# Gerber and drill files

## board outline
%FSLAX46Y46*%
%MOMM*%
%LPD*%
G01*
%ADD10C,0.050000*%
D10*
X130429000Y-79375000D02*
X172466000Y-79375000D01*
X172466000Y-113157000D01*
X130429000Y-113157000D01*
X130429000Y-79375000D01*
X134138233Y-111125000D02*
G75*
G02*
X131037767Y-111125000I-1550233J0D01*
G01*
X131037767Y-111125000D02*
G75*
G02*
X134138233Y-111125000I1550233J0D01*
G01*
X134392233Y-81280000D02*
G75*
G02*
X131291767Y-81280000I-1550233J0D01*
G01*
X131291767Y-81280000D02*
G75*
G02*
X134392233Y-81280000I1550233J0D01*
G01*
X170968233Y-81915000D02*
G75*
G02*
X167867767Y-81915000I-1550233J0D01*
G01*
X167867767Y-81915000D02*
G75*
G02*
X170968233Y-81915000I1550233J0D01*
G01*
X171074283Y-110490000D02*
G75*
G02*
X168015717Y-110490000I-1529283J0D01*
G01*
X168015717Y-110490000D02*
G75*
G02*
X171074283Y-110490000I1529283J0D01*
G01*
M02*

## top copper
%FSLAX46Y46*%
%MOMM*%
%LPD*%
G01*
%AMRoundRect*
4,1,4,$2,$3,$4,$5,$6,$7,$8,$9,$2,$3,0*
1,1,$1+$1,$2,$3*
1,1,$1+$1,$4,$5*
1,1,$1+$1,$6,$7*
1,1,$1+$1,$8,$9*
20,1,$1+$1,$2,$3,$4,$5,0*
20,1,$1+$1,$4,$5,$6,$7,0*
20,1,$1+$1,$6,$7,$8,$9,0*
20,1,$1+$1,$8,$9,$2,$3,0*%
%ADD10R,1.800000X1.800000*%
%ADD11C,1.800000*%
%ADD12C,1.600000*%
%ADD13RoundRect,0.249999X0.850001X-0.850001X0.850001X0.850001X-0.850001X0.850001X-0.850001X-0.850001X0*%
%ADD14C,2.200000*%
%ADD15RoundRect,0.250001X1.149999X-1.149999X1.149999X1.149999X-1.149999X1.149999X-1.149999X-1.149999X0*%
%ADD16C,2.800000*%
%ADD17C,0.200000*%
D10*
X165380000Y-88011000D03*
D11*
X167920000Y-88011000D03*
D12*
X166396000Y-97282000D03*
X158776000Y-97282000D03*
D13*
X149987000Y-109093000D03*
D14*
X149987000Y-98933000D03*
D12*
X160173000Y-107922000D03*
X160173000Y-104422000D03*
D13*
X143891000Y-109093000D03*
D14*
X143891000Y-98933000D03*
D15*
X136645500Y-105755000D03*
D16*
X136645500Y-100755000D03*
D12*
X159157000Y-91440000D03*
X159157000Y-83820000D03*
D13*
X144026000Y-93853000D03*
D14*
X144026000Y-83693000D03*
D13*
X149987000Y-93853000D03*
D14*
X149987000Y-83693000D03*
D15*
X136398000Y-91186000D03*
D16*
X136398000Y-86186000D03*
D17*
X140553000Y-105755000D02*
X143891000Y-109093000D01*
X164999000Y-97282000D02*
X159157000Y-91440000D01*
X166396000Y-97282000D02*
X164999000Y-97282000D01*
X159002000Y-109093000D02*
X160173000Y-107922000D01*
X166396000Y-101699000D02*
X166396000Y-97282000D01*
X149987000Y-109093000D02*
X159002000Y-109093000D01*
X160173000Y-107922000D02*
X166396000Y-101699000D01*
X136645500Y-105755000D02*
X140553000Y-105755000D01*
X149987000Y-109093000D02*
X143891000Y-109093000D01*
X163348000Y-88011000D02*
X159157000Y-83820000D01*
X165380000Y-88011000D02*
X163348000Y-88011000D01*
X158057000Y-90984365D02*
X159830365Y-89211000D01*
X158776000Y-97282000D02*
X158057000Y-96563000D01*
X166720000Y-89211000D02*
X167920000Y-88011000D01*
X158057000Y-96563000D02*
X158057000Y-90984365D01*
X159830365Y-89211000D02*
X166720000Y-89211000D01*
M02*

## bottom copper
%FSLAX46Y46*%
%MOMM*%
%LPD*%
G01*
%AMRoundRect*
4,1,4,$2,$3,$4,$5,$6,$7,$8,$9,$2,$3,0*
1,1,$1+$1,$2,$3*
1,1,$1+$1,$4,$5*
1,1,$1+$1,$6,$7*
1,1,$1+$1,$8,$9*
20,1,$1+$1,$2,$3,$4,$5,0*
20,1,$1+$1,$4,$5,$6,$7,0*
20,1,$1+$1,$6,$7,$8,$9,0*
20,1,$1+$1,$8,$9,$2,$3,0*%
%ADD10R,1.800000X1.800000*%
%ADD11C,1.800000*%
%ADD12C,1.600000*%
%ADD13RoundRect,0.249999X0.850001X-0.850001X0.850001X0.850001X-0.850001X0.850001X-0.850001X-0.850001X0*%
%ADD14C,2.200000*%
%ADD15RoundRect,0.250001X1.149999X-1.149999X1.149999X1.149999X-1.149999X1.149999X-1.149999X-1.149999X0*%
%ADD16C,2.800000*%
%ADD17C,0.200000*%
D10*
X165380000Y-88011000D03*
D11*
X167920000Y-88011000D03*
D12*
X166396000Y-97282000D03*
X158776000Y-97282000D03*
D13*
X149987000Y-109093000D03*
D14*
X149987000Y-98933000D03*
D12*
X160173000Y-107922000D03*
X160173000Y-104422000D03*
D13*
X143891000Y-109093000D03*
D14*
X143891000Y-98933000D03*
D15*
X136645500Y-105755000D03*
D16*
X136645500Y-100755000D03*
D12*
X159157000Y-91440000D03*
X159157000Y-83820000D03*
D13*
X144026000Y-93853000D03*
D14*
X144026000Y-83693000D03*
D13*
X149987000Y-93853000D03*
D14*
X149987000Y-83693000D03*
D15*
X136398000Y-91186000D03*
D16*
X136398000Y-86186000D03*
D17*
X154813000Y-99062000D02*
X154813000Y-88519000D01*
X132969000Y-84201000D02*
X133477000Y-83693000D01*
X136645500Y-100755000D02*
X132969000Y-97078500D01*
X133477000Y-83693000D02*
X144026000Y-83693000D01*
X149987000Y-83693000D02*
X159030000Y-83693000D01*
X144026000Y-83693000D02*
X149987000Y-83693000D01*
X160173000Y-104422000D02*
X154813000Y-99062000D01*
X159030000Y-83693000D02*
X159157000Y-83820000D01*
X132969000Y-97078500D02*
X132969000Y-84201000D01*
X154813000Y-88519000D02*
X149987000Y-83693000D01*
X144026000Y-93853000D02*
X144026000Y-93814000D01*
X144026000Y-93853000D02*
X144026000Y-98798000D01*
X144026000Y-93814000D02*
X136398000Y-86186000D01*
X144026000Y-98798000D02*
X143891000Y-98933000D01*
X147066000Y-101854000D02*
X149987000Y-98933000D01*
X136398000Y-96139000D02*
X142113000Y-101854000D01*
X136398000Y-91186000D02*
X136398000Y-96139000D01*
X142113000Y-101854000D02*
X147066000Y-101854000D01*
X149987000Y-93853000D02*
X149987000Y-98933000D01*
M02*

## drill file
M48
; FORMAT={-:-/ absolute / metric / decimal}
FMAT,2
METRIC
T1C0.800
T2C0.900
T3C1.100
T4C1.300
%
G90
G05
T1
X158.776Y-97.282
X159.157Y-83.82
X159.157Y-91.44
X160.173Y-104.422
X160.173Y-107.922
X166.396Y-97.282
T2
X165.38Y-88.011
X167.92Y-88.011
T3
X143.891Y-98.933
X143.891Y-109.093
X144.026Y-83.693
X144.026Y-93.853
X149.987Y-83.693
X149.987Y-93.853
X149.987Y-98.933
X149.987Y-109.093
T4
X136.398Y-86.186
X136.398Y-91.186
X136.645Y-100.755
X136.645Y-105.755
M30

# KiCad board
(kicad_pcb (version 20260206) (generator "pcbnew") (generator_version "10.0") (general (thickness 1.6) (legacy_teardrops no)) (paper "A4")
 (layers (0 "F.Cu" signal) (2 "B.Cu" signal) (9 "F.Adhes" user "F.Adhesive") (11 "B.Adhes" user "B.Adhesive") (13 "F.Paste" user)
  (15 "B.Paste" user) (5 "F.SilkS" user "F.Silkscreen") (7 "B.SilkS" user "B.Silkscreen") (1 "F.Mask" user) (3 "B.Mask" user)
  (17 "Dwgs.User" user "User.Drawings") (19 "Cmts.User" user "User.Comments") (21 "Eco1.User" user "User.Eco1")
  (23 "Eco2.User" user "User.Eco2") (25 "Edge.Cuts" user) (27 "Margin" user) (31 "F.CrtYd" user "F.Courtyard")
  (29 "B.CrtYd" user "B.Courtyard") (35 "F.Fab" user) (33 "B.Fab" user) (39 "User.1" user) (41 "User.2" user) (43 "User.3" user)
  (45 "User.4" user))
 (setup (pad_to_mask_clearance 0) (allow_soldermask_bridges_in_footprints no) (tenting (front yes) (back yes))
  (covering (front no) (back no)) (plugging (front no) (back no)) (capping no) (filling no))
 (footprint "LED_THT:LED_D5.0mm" (layer "F.Cu") (at 165.38 88.011)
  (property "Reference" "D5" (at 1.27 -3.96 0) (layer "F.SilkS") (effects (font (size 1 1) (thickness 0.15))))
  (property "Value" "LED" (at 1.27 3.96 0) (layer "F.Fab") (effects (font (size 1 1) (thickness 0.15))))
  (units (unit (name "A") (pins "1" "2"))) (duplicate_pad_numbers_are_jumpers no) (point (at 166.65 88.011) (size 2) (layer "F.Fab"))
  (pad "1" thru_hole rect (at 0 0) (size 1.8 1.8) (drill 0.9) (layers "*.Cu" "*.Mask") (remove_unused_layers no) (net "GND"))
  (pad "2" thru_hole circle (at 2.54 0) (size 1.8 1.8) (drill 0.9) (layers "*.Cu" "*.Mask") (remove_unused_layers no) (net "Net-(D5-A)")))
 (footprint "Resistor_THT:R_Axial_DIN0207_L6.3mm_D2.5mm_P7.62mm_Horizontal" (layer "F.Cu") (at 166.396 97.282 180)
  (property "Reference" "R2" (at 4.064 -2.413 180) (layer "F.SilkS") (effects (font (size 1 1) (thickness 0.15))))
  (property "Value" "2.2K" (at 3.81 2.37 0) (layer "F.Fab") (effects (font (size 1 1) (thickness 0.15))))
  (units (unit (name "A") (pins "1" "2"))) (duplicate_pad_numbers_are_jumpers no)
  (pad "1" thru_hole circle (at 0 0 180) (size 1.6 1.6) (drill 0.8) (layers "*.Cu" "*.Mask") (remove_unused_layers no) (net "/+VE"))
  (pad "2" thru_hole circle (at 7.62 0 180) (size 1.6 1.6) (drill 0.8) (layers "*.Cu" "*.Mask") (remove_unused_layers no) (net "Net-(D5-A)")))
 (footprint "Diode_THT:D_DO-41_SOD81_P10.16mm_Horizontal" (layer "F.Cu") (at 149.987 109.093 90)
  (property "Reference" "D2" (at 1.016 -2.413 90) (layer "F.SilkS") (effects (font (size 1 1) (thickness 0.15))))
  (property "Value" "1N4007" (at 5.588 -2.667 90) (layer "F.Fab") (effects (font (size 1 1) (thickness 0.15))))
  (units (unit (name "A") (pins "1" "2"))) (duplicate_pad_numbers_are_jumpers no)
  (pad "1" thru_hole roundrect (at 0 0 90) (size 2.2 2.2) (drill 1.1) (layers "*.Cu" "*.Mask") (remove_unused_layers no)
   (roundrect_rratio 0.113636) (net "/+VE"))
  (pad "2" thru_hole circle (at 10.16 0 90) (size 2.2 2.2) (drill 1.1) (layers "*.Cu" "*.Mask") (remove_unused_layers no) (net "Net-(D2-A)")))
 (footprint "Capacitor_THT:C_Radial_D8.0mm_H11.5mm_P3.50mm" (layer "F.Cu") (at 160.173 107.922 90)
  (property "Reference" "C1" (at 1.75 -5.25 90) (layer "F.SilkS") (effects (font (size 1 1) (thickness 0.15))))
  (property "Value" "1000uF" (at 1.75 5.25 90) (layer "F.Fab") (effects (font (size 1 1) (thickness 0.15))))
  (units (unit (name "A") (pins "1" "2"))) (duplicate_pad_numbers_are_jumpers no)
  (pad "1" thru_hole circle (at 0 0 90) (size 1.6 1.6) (drill 0.8) (layers "*.Cu" "*.Mask") (remove_unused_layers no) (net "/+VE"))
  (pad "2" thru_hole circle (at 3.5 0 90) (size 1.6 1.6) (drill 0.8) (layers "*.Cu" "*.Mask") (remove_unused_layers no) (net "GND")))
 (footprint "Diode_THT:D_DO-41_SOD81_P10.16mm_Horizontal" (layer "F.Cu") (at 143.891 109.093 90)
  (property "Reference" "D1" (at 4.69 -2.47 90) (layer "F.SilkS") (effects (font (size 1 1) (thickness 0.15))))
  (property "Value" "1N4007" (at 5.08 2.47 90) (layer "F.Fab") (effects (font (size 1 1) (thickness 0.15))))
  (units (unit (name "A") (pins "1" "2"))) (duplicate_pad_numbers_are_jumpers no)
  (pad "1" thru_hole roundrect (at 0 0 90) (size 2.2 2.2) (drill 1.1) (layers "*.Cu" "*.Mask") (remove_unused_layers no)
   (roundrect_rratio 0.113636) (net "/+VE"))
  (pad "2" thru_hole circle (at 10.16 0 90) (size 2.2 2.2) (drill 1.1) (layers "*.Cu" "*.Mask") (remove_unused_layers no) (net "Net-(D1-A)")))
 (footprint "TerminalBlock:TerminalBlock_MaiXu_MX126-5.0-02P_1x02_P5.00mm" (layer "F.Cu") (at 136.6455 105.755 90)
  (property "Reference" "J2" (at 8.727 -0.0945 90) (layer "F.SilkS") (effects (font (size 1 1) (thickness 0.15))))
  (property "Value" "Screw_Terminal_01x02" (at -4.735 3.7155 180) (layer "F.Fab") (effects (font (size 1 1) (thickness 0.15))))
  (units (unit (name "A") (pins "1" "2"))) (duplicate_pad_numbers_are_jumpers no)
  (pad "1" thru_hole roundrect (at 0 0 90) (size 2.8 2.8) (drill 1.3) (layers "*.Cu" "*.Mask") (remove_unused_layers no)
   (roundrect_rratio 0.089286) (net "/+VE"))
  (pad "2" thru_hole circle (at 5 0 90) (size 2.8 2.8) (drill 1.3) (layers "*.Cu" "*.Mask") (remove_unused_layers no) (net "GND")))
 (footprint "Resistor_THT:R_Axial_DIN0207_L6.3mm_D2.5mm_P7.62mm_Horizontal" (layer "F.Cu") (at 159.157 91.44 90)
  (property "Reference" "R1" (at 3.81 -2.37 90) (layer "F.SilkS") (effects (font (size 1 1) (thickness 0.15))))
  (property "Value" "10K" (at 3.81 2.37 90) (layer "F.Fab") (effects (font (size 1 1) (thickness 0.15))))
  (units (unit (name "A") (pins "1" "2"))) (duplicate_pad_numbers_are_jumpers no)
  (pad "1" thru_hole circle (at 0 0 90) (size 1.6 1.6) (drill 0.8) (layers "*.Cu" "*.Mask") (remove_unused_layers no) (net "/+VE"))
  (pad "2" thru_hole circle (at 7.62 0 90) (size 1.6 1.6) (drill 0.8) (layers "*.Cu" "*.Mask") (remove_unused_layers no) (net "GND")))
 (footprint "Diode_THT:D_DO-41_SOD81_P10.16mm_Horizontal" (layer "F.Cu") (at 144.026 93.853 90)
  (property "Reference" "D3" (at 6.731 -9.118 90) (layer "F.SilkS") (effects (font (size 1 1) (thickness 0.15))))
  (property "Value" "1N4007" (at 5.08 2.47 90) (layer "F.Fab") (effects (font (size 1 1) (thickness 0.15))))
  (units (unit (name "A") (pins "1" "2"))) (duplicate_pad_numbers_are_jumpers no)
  (pad "1" thru_hole roundrect (at 0 0 90) (size 2.2 2.2) (drill 1.1) (layers "*.Cu" "*.Mask") (remove_unused_layers no)
   (roundrect_rratio 0.113636) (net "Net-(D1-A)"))
  (pad "2" thru_hole circle (at 10.16 0 90) (size 2.2 2.2) (drill 1.1) (layers "*.Cu" "*.Mask") (remove_unused_layers no) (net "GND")))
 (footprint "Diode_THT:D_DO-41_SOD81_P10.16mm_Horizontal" (layer "F.Cu") (at 149.987 93.853 90)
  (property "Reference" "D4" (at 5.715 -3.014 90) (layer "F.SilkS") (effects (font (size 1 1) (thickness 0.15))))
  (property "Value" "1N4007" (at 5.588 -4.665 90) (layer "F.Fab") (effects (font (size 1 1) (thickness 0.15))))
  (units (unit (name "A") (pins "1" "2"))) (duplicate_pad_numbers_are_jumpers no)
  (pad "1" thru_hole roundrect (at 0 0 90) (size 2.2 2.2) (drill 1.1) (layers "*.Cu" "*.Mask") (remove_unused_layers no)
   (roundrect_rratio 0.113636) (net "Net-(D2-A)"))
  (pad "2" thru_hole circle (at 10.16 0 90) (size 2.2 2.2) (drill 1.1) (layers "*.Cu" "*.Mask") (remove_unused_layers no) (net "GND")))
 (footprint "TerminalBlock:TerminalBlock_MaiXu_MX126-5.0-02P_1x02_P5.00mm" (layer "F.Cu") (at 136.398 91.186 90)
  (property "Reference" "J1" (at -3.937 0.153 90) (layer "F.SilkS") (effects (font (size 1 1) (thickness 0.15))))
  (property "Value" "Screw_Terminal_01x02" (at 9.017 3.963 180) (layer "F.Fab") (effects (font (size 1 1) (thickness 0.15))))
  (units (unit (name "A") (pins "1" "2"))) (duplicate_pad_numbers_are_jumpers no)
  (pad "1" thru_hole roundrect (at 0 0 90) (size 2.8 2.8) (drill 1.3) (layers "*.Cu" "*.Mask") (remove_unused_layers no)
   (roundrect_rratio 0.089286) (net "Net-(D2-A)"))
  (pad "2" thru_hole circle (at 5 0 90) (size 2.8 2.8) (drill 1.3) (layers "*.Cu" "*.Mask") (remove_unused_layers no) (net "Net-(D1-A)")))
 (gr_rect (start 130.429 79.375) (end 172.466 113.157) (stroke (width 0.05) (type default)) (fill no) (layer "Edge.Cuts"))
 (gr_circle (center 132.588 111.125) (end 131.318 112.014) (stroke (width 0.05) (type default)) (fill no) (layer "Edge.Cuts"))
 (gr_circle (center 132.842 81.28) (end 131.572 80.391) (stroke (width 0.05) (type default)) (fill no) (layer "Edge.Cuts"))
 (gr_circle (center 169.418 81.915) (end 168.148 81.026) (stroke (width 0.05) (type default)) (fill no) (layer "Edge.Cuts"))
 (gr_circle (center 169.545 110.49) (end 170.688 111.506) (stroke (width 0.05) (type default)) (fill no) (layer "Edge.Cuts"))
 (segment (start 140.553 105.755) (end 143.891 109.093) (width 0.2) (layer "F.Cu") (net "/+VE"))
 (segment (start 164.999 97.282) (end 159.157 91.44) (width 0.2) (layer "F.Cu") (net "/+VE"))
 (segment (start 166.396 97.282) (end 164.999 97.282) (width 0.2) (layer "F.Cu") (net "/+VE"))
 (segment (start 159.002 109.093) (end 160.173 107.922) (width 0.2) (layer "F.Cu") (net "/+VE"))
 (segment (start 166.396 101.699) (end 166.396 97.282) (width 0.2) (layer "F.Cu") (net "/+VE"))
 (segment (start 149.987 109.093) (end 159.002 109.093) (width 0.2) (layer "F.Cu") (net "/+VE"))
 (segment (start 160.173 107.922) (end 166.396 101.699) (width 0.2) (layer "F.Cu") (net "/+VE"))
 (segment (start 136.6455 105.755) (end 140.553 105.755) (width 0.2) (layer "F.Cu") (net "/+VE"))
 (segment (start 149.987 109.093) (end 143.891 109.093) (width 0.2) (layer "F.Cu") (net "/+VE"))
 (segment (start 163.348 88.011) (end 159.157 83.82) (width 0.2) (layer "F.Cu") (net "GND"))
 (segment (start 165.38 88.011) (end 163.348 88.011) (width 0.2) (layer "F.Cu") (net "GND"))
 (segment (start 154.813 99.062) (end 154.813 88.519) (width 0.2) (layer "B.Cu") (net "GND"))
 (segment (start 132.969 84.201) (end 133.477 83.693) (width 0.2) (layer "B.Cu") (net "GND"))
 (segment (start 136.6455 100.755) (end 132.969 97.0785) (width 0.2) (layer "B.Cu") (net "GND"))
 (segment (start 133.477 83.693) (end 144.026 83.693) (width 0.2) (layer "B.Cu") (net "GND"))
 (segment (start 149.987 83.693) (end 159.03 83.693) (width 0.2) (layer "B.Cu") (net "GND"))
 (segment (start 144.026 83.693) (end 149.987 83.693) (width 0.2) (layer "B.Cu") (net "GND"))
 (segment (start 160.173 104.422) (end 154.813 99.062) (width 0.2) (layer "B.Cu") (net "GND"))
 (segment (start 159.03 83.693) (end 159.157 83.82) (width 0.2) (layer "B.Cu") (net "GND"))
 (segment (start 132.969 97.0785) (end 132.969 84.201) (width 0.2) (layer "B.Cu") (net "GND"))
 (segment (start 154.813 88.519) (end 149.987 83.693) (width 0.2) (layer "B.Cu") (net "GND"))
 (segment (start 144.026 93.853) (end 144.026 93.814) (width 0.2) (layer "B.Cu") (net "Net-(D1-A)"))
 (segment (start 144.026 93.853) (end 144.026 98.798) (width 0.2) (layer "B.Cu") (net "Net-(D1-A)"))
 (segment (start 144.026 93.814) (end 136.398 86.186) (width 0.2) (layer "B.Cu") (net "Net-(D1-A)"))
 (segment (start 144.026 98.798) (end 143.891 98.933) (width 0.2) (layer "B.Cu") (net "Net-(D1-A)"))
 (segment (start 147.066 101.854) (end 149.987 98.933) (width 0.2) (layer "B.Cu") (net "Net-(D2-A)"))
 (segment (start 136.398 96.139) (end 142.113 101.854) (width 0.2) (layer "B.Cu") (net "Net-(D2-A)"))
 (segment (start 136.398 91.186) (end 136.398 96.139) (width 0.2) (layer "B.Cu") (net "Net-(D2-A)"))
 (segment (start 142.113 101.854) (end 147.066 101.854) (width 0.2) (layer "B.Cu") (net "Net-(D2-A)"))
 (segment (start 149.987 93.853) (end 149.987 98.933) (width 0.2) (layer "B.Cu") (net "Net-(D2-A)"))
 (segment (start 158.057 90.984365) (end 159.830365 89.211) (width 0.2) (layer "F.Cu") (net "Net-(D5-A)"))
 (segment (start 158.776 97.282) (end 158.057 96.563) (width 0.2) (layer "F.Cu") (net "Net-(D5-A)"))
 (segment (start 166.72 89.211) (end 167.92 88.011) (width 0.2) (layer "F.Cu") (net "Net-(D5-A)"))
 (segment (start 158.057 96.563) (end 158.057 90.984365) (width 0.2) (layer "F.Cu") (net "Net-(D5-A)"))
 (segment (start 159.830365 89.211) (end 166.72 89.211) (width 0.2) (layer "F.Cu") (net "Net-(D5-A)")))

